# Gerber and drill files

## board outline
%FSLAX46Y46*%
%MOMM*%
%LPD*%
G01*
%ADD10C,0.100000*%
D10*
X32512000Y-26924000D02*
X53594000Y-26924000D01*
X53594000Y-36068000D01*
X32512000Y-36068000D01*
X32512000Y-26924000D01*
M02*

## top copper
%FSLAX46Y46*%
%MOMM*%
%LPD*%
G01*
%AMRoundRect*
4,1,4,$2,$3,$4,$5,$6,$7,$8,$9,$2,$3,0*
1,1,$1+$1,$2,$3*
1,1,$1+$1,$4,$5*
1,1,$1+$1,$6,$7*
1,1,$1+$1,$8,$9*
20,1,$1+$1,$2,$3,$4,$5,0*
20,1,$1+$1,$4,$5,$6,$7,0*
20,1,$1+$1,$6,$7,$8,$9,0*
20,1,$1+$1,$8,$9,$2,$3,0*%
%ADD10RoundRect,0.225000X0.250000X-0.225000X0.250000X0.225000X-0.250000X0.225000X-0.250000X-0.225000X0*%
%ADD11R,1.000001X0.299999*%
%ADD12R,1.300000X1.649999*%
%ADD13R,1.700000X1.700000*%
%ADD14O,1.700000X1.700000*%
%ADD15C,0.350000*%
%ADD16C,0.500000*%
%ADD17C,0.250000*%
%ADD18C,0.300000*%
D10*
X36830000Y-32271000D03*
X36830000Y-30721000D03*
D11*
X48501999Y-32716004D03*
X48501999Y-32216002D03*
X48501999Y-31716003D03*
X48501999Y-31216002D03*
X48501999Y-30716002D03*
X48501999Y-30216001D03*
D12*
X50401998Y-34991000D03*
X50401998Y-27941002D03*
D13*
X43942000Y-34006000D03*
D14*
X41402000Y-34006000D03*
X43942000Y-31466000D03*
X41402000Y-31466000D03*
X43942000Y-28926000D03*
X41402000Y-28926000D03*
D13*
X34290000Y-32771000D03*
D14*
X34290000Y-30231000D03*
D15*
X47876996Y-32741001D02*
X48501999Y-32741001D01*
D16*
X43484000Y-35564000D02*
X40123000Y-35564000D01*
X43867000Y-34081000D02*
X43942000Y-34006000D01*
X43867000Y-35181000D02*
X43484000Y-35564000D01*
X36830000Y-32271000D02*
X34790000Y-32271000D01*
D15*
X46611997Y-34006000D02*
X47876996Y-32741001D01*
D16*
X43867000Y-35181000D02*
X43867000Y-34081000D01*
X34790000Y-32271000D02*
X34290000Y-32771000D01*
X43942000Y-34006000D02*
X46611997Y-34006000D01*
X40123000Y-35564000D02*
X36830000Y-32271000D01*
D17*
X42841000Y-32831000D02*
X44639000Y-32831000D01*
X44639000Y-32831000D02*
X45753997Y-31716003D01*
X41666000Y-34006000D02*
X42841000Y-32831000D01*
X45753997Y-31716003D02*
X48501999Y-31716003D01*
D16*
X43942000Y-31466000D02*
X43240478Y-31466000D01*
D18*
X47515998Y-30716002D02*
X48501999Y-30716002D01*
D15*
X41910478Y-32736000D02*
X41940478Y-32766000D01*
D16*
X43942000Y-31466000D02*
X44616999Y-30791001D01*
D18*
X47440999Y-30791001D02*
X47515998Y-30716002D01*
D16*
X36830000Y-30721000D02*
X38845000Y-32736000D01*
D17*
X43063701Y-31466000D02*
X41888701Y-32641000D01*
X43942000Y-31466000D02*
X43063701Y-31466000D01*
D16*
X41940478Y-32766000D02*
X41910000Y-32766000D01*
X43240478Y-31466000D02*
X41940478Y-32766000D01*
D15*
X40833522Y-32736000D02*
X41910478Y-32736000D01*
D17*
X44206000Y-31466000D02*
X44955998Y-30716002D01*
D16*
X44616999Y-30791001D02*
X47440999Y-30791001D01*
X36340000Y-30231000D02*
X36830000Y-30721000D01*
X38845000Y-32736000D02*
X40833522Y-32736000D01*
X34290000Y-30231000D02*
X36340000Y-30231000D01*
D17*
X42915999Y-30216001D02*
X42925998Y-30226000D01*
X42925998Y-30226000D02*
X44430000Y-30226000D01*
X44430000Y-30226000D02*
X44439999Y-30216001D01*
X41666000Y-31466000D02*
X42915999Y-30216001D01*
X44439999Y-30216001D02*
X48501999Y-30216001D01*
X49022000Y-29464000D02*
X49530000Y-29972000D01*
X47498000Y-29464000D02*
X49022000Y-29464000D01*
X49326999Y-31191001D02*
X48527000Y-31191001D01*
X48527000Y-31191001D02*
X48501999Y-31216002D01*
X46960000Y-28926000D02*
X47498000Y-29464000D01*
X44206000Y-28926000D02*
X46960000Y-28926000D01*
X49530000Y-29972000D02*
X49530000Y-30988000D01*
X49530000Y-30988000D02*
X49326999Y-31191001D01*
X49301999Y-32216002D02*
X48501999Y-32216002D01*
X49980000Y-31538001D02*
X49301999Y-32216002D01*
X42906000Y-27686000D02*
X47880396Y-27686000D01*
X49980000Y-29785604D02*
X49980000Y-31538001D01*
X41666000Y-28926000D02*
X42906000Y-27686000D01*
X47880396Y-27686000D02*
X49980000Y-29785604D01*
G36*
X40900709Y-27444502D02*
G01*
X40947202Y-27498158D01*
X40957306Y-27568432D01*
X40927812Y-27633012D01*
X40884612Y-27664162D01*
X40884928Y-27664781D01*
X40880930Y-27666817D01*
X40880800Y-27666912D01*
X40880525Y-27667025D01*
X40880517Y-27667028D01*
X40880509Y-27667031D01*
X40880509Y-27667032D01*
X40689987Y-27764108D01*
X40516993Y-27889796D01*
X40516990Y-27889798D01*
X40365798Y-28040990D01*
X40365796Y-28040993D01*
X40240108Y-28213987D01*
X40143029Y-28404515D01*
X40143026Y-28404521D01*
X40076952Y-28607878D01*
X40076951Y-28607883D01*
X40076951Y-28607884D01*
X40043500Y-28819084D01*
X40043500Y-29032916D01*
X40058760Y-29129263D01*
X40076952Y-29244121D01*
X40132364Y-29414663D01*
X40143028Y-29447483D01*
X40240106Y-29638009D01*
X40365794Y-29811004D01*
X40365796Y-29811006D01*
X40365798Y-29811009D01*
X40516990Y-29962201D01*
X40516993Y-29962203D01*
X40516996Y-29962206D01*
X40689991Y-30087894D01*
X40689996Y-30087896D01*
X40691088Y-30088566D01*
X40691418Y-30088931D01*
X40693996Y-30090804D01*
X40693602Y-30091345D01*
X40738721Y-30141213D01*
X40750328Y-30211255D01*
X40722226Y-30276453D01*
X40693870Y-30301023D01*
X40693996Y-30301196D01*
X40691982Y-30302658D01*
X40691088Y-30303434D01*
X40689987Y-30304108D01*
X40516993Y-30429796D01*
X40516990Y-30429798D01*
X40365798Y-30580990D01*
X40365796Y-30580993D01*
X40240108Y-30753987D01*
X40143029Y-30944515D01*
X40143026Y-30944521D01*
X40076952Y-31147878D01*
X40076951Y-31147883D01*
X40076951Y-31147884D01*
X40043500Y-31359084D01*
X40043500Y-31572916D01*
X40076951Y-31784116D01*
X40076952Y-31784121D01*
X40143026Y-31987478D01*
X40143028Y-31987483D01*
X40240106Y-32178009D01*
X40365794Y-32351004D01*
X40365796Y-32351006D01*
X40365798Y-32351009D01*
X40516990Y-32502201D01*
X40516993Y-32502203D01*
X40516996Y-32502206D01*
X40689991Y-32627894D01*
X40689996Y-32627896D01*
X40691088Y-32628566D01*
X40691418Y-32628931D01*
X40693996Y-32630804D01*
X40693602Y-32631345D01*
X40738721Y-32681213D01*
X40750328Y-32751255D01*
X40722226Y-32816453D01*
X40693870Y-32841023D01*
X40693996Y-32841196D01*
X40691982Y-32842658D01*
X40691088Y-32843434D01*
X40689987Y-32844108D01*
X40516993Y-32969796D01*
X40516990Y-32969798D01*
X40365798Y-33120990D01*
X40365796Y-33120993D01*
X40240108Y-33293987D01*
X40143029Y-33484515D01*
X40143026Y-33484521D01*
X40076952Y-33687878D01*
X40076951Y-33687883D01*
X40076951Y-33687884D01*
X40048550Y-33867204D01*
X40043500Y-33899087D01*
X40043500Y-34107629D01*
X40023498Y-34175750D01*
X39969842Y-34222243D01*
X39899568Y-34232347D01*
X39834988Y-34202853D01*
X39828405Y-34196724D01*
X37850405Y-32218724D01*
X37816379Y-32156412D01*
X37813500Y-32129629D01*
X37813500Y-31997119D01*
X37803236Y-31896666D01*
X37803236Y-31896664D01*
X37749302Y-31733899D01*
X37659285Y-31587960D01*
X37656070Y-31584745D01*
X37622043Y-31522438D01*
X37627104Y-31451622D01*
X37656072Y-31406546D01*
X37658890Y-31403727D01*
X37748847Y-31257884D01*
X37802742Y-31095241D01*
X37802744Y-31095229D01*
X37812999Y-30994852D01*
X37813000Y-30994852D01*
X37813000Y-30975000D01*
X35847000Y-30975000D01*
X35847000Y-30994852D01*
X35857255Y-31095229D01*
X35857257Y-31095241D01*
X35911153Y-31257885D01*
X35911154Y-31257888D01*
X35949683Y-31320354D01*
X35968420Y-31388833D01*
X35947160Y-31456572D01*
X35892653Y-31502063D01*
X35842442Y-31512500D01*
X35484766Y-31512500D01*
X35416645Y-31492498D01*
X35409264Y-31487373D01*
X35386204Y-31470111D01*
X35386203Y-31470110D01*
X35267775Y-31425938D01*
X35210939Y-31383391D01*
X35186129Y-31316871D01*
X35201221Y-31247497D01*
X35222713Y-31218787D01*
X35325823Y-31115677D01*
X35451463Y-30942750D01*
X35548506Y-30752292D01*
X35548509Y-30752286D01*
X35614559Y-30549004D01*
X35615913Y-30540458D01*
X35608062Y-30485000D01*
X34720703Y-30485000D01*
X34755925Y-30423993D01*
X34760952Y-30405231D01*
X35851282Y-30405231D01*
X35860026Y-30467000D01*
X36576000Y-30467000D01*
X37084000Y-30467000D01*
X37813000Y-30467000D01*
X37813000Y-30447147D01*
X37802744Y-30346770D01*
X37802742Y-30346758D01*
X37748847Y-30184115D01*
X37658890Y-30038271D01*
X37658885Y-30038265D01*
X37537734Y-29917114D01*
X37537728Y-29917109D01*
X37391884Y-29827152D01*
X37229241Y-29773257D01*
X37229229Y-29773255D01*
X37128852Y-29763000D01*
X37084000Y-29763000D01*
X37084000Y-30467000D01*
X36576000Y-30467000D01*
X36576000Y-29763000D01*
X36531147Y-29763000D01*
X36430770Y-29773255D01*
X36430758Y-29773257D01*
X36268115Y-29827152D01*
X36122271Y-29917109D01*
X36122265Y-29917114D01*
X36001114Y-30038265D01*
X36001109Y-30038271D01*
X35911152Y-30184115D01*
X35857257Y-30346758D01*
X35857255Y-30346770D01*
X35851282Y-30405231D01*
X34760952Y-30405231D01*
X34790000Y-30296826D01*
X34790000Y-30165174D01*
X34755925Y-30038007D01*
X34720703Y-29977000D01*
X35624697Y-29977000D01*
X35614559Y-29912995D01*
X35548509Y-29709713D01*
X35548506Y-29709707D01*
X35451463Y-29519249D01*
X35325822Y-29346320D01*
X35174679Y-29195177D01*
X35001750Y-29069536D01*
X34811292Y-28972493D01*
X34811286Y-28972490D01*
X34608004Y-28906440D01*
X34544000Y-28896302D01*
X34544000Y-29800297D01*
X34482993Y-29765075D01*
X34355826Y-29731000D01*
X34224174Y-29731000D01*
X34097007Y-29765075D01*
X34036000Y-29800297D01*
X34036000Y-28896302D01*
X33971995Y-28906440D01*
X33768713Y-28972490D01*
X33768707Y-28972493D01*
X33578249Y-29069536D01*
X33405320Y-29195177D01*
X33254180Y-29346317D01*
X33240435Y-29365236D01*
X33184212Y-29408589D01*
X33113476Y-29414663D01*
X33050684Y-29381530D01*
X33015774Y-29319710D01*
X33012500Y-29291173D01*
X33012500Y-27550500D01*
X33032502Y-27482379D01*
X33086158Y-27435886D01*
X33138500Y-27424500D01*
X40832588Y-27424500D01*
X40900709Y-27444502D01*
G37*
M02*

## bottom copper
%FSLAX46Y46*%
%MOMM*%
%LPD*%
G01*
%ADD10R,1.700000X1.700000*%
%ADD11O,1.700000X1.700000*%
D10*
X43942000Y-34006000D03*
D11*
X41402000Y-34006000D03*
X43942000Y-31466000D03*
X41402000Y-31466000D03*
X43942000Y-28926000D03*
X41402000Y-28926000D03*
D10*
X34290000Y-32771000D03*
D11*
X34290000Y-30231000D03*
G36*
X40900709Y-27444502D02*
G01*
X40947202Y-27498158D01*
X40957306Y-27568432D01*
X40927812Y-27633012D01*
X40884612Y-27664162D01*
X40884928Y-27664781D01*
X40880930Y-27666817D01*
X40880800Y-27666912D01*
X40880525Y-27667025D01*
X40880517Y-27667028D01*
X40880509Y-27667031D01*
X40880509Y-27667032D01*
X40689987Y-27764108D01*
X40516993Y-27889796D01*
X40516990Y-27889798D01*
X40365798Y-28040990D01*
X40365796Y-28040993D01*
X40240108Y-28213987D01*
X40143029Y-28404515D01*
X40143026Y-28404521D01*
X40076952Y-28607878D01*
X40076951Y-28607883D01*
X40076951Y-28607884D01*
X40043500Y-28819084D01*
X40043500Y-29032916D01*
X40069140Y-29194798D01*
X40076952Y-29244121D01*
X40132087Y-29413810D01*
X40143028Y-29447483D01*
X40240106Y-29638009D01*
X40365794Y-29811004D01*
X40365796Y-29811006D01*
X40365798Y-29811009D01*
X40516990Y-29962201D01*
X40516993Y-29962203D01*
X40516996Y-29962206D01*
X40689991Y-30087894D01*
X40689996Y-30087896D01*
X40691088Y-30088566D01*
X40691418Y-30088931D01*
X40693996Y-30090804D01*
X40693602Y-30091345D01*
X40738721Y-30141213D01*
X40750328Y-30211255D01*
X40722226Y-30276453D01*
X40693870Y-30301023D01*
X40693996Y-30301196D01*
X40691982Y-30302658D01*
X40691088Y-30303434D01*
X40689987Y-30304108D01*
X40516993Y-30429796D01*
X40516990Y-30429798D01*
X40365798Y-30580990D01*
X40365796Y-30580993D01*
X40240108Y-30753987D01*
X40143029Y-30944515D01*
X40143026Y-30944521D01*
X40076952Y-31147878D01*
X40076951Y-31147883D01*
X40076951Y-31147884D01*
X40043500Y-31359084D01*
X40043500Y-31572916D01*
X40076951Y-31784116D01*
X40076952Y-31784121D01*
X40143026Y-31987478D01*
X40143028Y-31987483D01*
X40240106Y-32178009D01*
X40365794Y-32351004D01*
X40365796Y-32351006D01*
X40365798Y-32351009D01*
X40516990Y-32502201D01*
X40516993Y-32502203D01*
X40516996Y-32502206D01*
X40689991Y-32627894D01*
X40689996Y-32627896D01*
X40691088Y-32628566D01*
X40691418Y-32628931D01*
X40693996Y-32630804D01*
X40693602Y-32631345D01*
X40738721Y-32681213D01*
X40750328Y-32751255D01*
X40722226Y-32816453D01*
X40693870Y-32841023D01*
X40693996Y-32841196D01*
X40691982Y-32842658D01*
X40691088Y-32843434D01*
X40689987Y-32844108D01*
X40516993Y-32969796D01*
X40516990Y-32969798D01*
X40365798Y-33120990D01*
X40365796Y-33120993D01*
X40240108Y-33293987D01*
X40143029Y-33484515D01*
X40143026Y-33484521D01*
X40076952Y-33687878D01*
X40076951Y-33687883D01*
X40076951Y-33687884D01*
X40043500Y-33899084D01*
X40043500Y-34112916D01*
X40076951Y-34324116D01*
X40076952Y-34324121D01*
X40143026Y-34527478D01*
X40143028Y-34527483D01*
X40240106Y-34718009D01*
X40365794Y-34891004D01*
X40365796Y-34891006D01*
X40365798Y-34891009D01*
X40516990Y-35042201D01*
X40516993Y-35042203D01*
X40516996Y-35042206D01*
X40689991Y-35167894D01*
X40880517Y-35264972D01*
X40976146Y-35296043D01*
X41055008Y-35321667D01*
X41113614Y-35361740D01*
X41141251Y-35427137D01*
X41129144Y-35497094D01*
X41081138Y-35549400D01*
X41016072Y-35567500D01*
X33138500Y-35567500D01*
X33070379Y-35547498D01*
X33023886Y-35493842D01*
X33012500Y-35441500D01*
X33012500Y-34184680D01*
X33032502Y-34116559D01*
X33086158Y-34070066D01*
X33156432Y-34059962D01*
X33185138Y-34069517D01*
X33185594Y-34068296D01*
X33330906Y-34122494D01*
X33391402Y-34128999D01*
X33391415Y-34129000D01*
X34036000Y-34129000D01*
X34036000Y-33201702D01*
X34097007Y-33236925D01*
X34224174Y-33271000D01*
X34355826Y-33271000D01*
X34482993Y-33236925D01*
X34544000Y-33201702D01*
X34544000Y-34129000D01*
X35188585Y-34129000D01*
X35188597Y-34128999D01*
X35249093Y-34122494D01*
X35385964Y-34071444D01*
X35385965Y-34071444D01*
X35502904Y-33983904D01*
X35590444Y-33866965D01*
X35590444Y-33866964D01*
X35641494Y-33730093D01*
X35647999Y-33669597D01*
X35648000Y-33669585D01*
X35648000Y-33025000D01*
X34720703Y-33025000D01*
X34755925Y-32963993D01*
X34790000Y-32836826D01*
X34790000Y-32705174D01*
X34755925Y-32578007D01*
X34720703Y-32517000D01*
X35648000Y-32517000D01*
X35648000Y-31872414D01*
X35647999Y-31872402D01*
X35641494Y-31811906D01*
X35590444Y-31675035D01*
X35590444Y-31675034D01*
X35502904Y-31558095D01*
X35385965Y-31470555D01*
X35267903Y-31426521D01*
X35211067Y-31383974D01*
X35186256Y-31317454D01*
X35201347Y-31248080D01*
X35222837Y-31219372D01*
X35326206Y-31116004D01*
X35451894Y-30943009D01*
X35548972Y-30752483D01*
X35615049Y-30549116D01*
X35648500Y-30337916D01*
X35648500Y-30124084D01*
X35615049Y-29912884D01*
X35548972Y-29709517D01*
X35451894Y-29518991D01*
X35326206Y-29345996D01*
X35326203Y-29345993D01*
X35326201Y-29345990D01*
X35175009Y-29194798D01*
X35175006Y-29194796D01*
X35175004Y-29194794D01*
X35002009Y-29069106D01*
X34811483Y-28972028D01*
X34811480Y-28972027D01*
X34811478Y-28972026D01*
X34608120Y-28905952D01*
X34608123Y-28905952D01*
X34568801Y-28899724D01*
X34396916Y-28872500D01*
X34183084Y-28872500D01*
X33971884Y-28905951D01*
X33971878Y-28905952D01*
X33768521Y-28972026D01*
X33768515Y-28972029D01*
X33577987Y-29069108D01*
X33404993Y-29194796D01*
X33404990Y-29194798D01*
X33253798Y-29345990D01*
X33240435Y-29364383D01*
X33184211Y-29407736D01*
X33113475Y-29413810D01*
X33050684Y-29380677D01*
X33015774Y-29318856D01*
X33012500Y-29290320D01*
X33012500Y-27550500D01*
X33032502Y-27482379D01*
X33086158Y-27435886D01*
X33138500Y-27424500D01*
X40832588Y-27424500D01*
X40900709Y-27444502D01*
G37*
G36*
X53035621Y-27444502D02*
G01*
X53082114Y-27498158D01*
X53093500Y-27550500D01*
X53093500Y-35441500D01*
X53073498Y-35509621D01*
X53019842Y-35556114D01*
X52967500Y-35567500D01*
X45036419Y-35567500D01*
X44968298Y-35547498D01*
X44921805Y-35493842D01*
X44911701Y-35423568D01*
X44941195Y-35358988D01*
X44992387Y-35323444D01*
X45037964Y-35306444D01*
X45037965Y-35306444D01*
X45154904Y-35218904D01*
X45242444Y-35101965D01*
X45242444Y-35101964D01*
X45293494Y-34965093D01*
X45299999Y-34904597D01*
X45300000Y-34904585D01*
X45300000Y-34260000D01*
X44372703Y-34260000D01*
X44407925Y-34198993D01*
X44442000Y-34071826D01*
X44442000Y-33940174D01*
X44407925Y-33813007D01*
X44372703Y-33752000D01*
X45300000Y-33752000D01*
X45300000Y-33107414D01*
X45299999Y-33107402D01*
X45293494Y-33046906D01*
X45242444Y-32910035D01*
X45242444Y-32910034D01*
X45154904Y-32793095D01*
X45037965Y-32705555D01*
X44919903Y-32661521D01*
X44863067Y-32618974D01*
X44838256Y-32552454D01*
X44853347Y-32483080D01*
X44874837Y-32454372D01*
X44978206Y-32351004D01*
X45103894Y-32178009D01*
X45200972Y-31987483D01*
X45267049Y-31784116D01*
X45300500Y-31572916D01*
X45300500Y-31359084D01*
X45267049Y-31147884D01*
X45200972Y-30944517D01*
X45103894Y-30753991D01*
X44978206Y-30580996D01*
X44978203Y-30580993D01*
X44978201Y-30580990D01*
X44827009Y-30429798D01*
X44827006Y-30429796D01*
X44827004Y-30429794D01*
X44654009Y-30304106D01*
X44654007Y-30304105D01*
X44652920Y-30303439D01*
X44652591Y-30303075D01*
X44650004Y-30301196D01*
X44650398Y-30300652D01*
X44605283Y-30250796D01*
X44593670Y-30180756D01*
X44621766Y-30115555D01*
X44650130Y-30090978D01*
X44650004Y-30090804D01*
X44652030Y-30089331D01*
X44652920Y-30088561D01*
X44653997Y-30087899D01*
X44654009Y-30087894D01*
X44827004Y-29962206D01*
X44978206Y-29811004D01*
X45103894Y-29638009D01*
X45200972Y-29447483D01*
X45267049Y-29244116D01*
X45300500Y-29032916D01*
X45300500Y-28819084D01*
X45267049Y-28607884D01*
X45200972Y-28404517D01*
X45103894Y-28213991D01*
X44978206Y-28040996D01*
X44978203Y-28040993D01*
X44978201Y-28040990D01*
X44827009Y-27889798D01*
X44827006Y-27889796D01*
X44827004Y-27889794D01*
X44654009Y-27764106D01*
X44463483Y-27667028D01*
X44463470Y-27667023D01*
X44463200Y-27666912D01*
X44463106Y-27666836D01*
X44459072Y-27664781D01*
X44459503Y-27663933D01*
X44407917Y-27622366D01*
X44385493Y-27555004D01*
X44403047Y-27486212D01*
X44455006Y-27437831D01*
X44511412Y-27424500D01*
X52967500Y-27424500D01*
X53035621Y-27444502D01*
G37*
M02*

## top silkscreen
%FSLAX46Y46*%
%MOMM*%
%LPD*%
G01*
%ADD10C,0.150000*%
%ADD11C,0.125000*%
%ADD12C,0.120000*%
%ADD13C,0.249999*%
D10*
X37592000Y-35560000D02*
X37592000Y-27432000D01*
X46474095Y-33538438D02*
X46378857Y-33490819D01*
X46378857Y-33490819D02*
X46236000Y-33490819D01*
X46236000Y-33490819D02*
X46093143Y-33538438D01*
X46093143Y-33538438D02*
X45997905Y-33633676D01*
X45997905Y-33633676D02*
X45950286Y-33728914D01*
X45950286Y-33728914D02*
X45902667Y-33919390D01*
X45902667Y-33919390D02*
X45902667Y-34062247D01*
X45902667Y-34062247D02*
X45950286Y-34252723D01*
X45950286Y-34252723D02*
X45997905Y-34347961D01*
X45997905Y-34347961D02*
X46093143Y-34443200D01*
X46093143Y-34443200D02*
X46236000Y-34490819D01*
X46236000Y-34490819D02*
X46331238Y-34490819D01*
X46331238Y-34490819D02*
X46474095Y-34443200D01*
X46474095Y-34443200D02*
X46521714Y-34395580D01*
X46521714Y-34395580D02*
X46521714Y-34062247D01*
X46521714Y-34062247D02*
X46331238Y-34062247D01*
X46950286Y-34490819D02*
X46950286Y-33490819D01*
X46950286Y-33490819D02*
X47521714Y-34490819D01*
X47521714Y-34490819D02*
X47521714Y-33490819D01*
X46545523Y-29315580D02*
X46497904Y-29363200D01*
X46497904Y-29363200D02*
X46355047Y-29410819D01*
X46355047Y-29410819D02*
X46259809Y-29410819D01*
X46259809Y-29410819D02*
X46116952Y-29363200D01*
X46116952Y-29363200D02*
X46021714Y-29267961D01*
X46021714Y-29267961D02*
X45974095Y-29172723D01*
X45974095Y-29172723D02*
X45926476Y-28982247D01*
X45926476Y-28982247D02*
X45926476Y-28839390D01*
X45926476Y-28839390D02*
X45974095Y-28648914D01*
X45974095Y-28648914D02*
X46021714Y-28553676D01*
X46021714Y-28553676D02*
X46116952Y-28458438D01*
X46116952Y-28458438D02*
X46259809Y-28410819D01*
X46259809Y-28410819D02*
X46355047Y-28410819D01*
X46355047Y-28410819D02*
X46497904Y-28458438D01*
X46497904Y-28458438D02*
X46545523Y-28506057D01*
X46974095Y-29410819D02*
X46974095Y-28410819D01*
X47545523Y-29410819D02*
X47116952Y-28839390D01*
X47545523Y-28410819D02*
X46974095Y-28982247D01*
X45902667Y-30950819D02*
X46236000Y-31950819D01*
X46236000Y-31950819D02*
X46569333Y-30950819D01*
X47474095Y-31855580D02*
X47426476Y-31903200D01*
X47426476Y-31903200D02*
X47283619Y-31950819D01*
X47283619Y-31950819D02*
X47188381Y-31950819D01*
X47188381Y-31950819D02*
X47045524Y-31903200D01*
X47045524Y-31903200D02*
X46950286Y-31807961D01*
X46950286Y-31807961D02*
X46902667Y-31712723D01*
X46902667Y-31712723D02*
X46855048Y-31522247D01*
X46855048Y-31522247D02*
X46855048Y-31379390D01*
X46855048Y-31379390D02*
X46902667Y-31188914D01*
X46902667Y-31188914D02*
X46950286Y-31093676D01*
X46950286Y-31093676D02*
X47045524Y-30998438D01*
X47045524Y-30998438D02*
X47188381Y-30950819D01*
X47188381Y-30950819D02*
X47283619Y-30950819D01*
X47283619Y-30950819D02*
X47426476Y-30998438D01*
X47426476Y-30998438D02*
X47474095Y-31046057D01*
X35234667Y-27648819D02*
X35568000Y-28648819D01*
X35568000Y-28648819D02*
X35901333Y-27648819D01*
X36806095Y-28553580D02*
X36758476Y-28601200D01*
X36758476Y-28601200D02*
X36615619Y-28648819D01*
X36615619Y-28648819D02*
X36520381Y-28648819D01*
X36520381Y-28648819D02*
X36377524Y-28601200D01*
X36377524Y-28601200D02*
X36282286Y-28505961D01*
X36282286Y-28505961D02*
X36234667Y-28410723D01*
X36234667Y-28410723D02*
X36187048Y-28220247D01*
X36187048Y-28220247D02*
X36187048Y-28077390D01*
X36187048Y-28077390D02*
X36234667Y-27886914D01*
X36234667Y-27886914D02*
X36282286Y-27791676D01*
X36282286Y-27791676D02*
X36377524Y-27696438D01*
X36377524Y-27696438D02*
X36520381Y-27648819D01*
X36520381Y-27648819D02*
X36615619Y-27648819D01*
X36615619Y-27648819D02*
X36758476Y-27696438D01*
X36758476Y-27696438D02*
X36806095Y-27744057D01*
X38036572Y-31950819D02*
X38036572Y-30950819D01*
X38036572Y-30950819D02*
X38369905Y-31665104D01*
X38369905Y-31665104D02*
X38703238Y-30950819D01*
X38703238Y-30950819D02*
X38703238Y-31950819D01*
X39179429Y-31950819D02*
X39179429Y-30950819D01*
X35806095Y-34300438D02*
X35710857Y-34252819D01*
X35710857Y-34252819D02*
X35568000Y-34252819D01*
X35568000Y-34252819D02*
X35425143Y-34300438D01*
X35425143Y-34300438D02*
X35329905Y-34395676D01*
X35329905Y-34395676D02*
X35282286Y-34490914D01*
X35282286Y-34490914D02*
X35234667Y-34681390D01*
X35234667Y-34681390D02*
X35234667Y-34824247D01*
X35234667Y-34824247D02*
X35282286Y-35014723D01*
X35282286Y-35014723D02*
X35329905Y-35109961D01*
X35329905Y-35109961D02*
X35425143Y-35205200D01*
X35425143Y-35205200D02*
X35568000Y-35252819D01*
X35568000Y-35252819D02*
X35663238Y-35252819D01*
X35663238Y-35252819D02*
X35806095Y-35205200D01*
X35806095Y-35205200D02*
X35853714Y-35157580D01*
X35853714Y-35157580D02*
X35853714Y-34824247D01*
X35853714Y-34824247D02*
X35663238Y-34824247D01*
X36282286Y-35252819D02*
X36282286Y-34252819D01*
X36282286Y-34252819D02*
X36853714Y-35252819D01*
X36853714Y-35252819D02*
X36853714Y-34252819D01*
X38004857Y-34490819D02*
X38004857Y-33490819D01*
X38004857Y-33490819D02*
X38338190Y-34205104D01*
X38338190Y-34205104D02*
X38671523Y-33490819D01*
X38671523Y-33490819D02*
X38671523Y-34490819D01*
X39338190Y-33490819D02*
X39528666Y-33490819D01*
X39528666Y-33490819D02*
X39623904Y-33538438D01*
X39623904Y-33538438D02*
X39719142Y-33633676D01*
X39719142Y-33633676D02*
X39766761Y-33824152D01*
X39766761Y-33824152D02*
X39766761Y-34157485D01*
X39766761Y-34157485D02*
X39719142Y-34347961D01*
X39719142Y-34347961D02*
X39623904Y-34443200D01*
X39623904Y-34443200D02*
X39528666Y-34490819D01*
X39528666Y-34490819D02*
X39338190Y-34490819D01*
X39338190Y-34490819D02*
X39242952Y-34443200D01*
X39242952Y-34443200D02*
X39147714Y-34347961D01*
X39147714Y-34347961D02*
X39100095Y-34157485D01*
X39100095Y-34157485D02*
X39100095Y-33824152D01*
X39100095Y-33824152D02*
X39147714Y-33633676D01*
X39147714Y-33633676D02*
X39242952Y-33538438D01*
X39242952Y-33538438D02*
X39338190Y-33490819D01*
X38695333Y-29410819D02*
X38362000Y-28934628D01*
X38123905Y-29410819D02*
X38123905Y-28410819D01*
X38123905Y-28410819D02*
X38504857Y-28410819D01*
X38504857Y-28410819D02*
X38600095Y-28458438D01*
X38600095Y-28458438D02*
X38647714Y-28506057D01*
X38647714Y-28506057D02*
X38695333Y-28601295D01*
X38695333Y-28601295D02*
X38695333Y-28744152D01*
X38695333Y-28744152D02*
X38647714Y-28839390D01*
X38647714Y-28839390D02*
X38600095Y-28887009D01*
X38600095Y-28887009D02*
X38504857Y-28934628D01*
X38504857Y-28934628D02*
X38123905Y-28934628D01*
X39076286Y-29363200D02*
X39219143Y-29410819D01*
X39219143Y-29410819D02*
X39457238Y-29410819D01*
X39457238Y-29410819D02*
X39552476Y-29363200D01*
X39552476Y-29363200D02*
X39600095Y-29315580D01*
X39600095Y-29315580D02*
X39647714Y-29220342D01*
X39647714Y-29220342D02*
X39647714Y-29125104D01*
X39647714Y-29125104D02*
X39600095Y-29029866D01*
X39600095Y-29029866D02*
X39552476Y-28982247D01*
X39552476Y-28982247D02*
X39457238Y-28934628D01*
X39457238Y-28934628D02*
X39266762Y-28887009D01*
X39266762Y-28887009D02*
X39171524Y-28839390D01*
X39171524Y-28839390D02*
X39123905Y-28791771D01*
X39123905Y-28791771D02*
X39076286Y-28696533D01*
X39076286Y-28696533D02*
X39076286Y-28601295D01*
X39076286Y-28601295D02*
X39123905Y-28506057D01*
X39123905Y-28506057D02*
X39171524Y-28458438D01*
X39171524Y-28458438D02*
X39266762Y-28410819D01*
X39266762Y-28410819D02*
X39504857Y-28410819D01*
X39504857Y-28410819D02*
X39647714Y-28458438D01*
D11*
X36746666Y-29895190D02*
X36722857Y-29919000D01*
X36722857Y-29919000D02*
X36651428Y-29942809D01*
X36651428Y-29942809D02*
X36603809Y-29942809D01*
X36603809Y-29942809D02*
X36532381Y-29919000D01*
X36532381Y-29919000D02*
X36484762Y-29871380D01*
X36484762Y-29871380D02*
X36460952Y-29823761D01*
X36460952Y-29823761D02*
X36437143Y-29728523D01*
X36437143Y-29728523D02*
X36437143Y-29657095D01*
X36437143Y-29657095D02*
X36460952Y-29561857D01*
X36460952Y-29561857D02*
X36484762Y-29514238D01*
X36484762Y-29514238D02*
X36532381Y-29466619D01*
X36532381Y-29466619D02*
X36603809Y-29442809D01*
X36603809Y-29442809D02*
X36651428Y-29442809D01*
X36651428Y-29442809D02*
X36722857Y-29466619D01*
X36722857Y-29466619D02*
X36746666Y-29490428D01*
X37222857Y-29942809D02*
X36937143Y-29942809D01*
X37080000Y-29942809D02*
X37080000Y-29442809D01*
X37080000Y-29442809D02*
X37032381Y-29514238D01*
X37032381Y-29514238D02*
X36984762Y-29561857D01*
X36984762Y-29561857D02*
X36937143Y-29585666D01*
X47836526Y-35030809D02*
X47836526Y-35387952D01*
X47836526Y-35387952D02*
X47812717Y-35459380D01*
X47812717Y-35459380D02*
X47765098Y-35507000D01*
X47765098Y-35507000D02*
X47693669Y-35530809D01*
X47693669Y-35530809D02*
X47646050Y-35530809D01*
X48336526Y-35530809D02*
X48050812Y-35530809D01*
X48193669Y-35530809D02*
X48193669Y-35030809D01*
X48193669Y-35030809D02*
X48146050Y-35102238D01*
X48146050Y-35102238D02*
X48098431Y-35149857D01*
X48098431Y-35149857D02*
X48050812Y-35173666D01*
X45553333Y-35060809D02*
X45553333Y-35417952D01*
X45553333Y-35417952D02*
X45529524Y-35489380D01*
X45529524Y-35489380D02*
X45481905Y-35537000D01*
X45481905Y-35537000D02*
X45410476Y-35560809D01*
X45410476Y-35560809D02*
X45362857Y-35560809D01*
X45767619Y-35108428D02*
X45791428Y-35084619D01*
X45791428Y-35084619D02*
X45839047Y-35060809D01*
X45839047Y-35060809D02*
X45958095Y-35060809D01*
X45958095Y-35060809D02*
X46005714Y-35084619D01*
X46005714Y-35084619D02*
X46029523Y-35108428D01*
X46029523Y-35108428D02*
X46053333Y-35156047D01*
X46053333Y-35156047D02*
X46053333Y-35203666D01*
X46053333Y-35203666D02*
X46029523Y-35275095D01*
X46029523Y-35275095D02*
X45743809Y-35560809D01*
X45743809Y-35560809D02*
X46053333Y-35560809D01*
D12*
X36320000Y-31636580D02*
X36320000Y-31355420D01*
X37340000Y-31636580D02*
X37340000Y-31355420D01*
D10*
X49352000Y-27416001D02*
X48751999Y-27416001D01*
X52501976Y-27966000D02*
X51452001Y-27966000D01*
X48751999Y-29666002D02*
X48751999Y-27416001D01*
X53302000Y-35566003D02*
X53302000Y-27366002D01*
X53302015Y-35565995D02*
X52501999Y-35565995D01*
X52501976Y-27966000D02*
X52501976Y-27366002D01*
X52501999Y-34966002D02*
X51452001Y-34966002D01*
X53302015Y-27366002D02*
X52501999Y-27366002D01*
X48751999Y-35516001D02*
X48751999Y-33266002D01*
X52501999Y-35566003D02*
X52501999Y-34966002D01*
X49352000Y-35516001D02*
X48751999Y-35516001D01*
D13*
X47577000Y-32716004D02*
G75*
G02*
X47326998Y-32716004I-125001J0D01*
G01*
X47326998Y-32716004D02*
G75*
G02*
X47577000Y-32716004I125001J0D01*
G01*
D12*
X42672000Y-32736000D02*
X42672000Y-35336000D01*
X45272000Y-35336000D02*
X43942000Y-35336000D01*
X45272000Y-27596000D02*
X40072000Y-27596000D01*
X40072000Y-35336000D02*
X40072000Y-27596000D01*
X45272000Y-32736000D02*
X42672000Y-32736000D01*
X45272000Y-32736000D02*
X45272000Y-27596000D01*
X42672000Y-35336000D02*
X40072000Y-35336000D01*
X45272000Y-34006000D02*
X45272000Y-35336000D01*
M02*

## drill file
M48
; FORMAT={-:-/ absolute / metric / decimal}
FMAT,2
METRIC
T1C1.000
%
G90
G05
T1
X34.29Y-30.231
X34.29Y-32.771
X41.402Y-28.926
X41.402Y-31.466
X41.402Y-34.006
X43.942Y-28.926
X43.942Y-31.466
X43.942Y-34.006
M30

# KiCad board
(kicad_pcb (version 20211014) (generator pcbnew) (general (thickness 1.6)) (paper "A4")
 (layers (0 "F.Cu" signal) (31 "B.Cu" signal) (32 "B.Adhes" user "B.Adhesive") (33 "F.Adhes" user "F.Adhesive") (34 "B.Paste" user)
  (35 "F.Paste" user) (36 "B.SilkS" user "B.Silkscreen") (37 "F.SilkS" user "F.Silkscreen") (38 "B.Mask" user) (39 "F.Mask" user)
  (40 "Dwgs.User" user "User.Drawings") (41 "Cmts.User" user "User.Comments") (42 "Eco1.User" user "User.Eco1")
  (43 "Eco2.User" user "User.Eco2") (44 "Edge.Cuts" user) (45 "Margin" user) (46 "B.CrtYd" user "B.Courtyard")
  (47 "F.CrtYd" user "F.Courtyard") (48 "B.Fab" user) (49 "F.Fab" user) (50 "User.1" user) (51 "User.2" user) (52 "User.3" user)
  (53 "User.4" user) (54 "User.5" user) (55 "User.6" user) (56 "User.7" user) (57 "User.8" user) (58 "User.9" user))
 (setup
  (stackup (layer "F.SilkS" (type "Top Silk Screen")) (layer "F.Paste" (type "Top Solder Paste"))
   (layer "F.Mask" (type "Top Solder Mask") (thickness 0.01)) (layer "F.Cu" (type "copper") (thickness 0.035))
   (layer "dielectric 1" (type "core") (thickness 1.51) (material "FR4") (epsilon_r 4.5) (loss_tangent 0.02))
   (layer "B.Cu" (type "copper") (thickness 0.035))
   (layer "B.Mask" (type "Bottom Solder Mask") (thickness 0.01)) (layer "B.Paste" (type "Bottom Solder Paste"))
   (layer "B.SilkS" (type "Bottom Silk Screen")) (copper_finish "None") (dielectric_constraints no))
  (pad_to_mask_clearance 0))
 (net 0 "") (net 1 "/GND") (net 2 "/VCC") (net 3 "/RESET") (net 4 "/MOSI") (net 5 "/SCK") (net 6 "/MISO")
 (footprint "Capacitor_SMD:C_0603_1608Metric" (layer "F.Cu") (at 36.83 31.496 90)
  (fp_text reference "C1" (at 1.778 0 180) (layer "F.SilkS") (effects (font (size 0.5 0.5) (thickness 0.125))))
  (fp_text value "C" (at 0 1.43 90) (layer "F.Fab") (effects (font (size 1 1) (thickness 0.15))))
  (fp_line (start -0.14058 -0.51) (end 0.14058 -0.51) (layer "F.SilkS") (width 0.12))
  (fp_line (start -0.14058 0.51) (end 0.14058 0.51) (layer "F.SilkS") (width 0.12))
  (pad "1" smd roundrect (at -0.775 0 90) (size 0.9 0.95) (layers "F.Cu" "F.Paste" "F.Mask") (roundrect_rratio 0.25) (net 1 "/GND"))
  (pad "2" smd roundrect (at 0.775 0 90) (size 0.9 0.95) (layers "F.Cu" "F.Paste" "F.Mask") (roundrect_rratio 0.25) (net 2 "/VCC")))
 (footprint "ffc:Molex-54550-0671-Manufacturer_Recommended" (layer "F.Cu") (at 49.452 31.466001 90)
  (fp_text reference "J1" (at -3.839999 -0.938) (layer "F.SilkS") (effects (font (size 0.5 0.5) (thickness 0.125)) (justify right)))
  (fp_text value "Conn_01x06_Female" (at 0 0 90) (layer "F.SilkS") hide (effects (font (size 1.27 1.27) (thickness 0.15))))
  (fp_line (start 4.05 -0.1) (end 4.05 -0.700001) (layer "F.SilkS") (width 0.15))
  (fp_line (start 3.500001 3.049976) (end 3.500001 2.000001) (layer "F.SilkS") (width 0.15))
  (fp_line (start 1.799999 -0.700001) (end 4.05 -0.700001) (layer "F.SilkS") (width 0.15))
  (fp_line (start -4.100002 3.85) (end 4.099999 3.85) (layer "F.SilkS") (width 0.15))
  (fp_line (start -4.099994 3.850015) (end -4.099994 3.049999) (layer "F.SilkS") (width 0.15))
  (fp_line (start 3.500001 3.049976) (end 4.099999 3.049976) (layer "F.SilkS") (width 0.15))
  (fp_line (start -3.500001 3.049999) (end -3.500001 2.000001) (layer "F.SilkS") (width 0.15))
  (fp_line (start 4.099999 3.850015) (end 4.099999 3.049999) (layer "F.SilkS") (width 0.15))
  (fp_line (start -4.05 -0.700001) (end -1.800001 -0.700001) (layer "F.SilkS") (width 0.15))
  (fp_line (start -4.100002 3.049999) (end -3.500001 3.049999) (layer "F.SilkS") (width 0.15))
  (fp_line (start -4.05 -0.1) (end -4.05 -0.700001) (layer "F.SilkS") (width 0.15))
  (fp_circle (center -1.250003 -2.000001) (end -1.125002 -2.000001) (layer "F.SilkS") (width 0.249999) (fill none))
  (pad "1" smd rect locked (at -1.250003 -0.950001 90) (size 0.299999 1.000001) (layers "F.Cu" "F.Paste" "F.Mask") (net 1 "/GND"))
  (pad "2" smd rect locked (at -0.750001 -0.950001 90) (size 0.299999 1.000001) (layers "F.Cu" "F.Paste" "F.Mask") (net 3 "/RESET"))
  (pad "3" smd rect locked (at -0.250002 -0.950001 90) (size 0.299999 1.000001) (layers "F.Cu" "F.Paste" "F.Mask") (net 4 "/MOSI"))
  (pad "4" smd rect locked (at 0.249999 -0.950001 90) (size 0.299999 1.000001) (layers "F.Cu" "F.Paste" "F.Mask") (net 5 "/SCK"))
  (pad "5" smd rect locked (at 0.749999 -0.950001 90) (size 0.299999 1.000001) (layers "F.Cu" "F.Paste" "F.Mask") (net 2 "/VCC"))
  (pad "6" smd rect locked (at 1.25 -0.950001 90) (size 0.299999 1.000001) (layers "F.Cu" "F.Paste" "F.Mask") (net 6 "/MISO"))
  (pad "MP1" smd rect locked (at -3.524999 0.949998 90) (size 1.649999 1.3) (layers "F.Cu" "F.Paste" "F.Mask"))
  (pad "MP2" smd rect locked (at 3.524999 0.949998 90) (size 1.649999 1.3) (layers "F.Cu" "F.Paste" "F.Mask")))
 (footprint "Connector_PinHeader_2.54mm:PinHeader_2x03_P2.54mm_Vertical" (layer "F.Cu") (at 43.942 34.006 180)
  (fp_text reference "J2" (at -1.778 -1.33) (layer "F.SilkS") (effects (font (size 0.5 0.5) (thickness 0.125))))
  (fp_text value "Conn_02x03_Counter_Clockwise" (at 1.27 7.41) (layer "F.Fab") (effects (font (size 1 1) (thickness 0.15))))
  (fp_line (start 1.27 1.27) (end 1.27 -1.33) (layer "F.SilkS") (width 0.12))
  (fp_line (start -1.33 -1.33) (end 0 -1.33) (layer "F.SilkS") (width 0.12))
  (fp_line (start -1.33 6.41) (end 3.87 6.41) (layer "F.SilkS") (width 0.12))
  (fp_line (start 3.87 -1.33) (end 3.87 6.41) (layer "F.SilkS") (width 0.12))
  (fp_line (start -1.33 1.27) (end 1.27 1.27) (layer "F.SilkS") (width 0.12))
  (fp_line (start -1.33 1.27) (end -1.33 6.41) (layer "F.SilkS") (width 0.12))
  (fp_line (start 1.27 -1.33) (end 3.87 -1.33) (layer "F.SilkS") (width 0.12))
  (fp_line (start -1.33 0) (end -1.33 -1.33) (layer "F.SilkS") (width 0.12))
  (pad "1" thru_hole rect (at 0 0 180) (size 1.7 1.7) (drill 1) (layers *.Cu *.Mask) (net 1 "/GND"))
  (pad "2" thru_hole oval (at 2.54 0 180) (size 1.7 1.7) (drill 1) (layers *.Cu *.Mask) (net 4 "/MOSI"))
  (pad "3" thru_hole oval (at 0 2.54 180) (size 1.7 1.7) (drill 1) (layers *.Cu *.Mask) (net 2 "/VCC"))
  (pad "4" thru_hole oval (at 2.54 2.54 180) (size 1.7 1.7) (drill 1) (layers *.Cu *.Mask) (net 6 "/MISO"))
  (pad "5" thru_hole oval (at 0 5.08 180) (size 1.7 1.7) (drill 1) (layers *.Cu *.Mask) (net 5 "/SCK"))
  (pad "6" thru_hole oval (at 2.54 5.08 180) (size 1.7 1.7) (drill 1) (layers *.Cu *.Mask) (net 3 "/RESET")))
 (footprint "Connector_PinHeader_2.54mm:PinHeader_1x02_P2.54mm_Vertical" (layer "B.Cu") (at 34.29 32.771)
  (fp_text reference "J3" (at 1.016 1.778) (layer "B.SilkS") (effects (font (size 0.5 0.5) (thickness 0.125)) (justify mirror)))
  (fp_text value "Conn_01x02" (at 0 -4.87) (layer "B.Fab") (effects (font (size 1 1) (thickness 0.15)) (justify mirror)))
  (pad "1" thru_hole rect (at 0 0) (size 1.7 1.7) (drill 1) (layers *.Cu *.Mask) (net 1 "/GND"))
  (pad "2" thru_hole oval (at 0 -2.54) (size 1.7 1.7) (drill 1) (layers *.Cu *.Mask) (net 2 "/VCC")))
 (gr_line (start 37.592 35.56) (end 37.592 27.432) (layer "F.SilkS") (width 0.15))
 (gr_rect (start 32.512 26.924) (end 53.594 36.068) (layer "Edge.Cuts") (width 0.1) (fill none))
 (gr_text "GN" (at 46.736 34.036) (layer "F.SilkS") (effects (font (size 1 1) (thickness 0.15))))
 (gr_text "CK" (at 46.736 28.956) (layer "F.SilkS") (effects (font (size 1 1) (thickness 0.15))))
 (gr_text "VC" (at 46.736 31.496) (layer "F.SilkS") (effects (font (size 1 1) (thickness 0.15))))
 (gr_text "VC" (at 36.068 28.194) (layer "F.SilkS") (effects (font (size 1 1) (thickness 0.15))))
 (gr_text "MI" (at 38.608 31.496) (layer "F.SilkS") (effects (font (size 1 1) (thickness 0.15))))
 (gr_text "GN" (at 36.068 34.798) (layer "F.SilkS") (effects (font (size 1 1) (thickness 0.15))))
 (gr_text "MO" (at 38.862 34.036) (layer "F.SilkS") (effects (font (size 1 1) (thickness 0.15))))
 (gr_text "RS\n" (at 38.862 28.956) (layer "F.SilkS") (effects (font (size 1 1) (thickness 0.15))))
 (segment (start 47.876996 32.741001) (end 48.501999 32.741001) (width 0.35) (layer "F.Cu") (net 1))
 (segment (start 43.484 35.564) (end 40.123 35.564) (width 0.5) (layer "F.Cu") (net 1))
 (segment (start 43.867 34.081) (end 43.942 34.006) (width 0.5) (layer "F.Cu") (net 1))
 (segment (start 43.867 35.181) (end 43.484 35.564) (width 0.5) (layer "F.Cu") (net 1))
 (segment (start 36.83 32.271) (end 34.79 32.271) (width 0.5) (layer "F.Cu") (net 1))
 (segment (start 46.611997 34.006) (end 47.876996 32.741001) (width 0.35) (layer "F.Cu") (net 1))
 (segment (start 43.867 35.181) (end 43.867 34.081) (width 0.5) (layer "F.Cu") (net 1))
 (segment (start 34.79 32.271) (end 34.29 32.771) (width 0.5) (layer "F.Cu") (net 1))
 (segment (start 43.942 34.006) (end 46.611997 34.006) (width 0.5) (layer "F.Cu") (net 1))
 (segment (start 40.123 35.564) (end 36.83 32.271) (width 0.5) (layer "F.Cu") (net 1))
 (segment (start 42.841 32.831) (end 44.639 32.831) (width 0.25) (layer "F.Cu") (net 4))
 (segment (start 44.639 32.831) (end 45.753997 31.716003) (width 0.25) (layer "F.Cu") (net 4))
 (segment (start 41.666 34.006) (end 42.841 32.831) (width 0.25) (layer "F.Cu") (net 4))
 (segment (start 45.753997 31.716003) (end 48.501999 31.716003) (width 0.25) (layer "F.Cu") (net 4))
 (segment (start 43.942 31.466) (end 43.240478 31.466) (width 0.5) (layer "F.Cu") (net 2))
 (segment (start 47.515998 30.716002) (end 48.501999 30.716002) (width 0.3) (layer "F.Cu") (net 2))
 (segment (start 41.910478 32.736) (end 41.940478 32.766) (width 0.35) (layer "F.Cu") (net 2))
 (segment (start 43.942 31.466) (end 44.616999 30.791001) (width 0.5) (layer "F.Cu") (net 2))
 (segment (start 47.440999 30.791001) (end 47.515998 30.716002) (width 0.3) (layer "F.Cu") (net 2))
 (segment (start 36.83 30.721) (end 38.845 32.736) (width 0.5) (layer "F.Cu") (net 2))
 (segment (start 43.063701 31.466) (end 41.888701 32.641) (width 0.25) (layer "F.Cu") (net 2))
 (segment (start 43.942 31.466) (end 43.063701 31.466) (width 0.25) (layer "F.Cu") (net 2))
 (segment (start 41.940478 32.766) (end 41.91 32.766) (width 0.5) (layer "F.Cu") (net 2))
 (segment (start 43.240478 31.466) (end 41.940478 32.766) (width 0.5) (layer "F.Cu") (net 2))
 (segment (start 40.833522 32.736) (end 41.910478 32.736) (width 0.35) (layer "F.Cu") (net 2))
 (segment (start 44.206 31.466) (end 44.955998 30.716002) (width 0.25) (layer "F.Cu") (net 2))
 (segment (start 44.616999 30.791001) (end 47.440999 30.791001) (width 0.5) (layer "F.Cu") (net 2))
 (segment (start 36.34 30.231) (end 36.83 30.721) (width 0.5) (layer "F.Cu") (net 2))
 (segment (start 38.845 32.736) (end 40.833522 32.736) (width 0.5) (layer "F.Cu") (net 2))
 (segment (start 34.29 30.231) (end 36.34 30.231) (width 0.5) (layer "F.Cu") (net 2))
 (segment (start 42.915999 30.216001) (end 42.925998 30.226) (width 0.25) (layer "F.Cu") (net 6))
 (segment (start 42.925998 30.226) (end 44.43 30.226) (width 0.25) (layer "F.Cu") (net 6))
 (segment (start 44.43 30.226) (end 44.439999 30.216001) (width 0.25) (layer "F.Cu") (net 6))
 (segment (start 41.666 31.466) (end 42.915999 30.216001) (width 0.25) (layer "F.Cu") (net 6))
 (segment (start 44.439999 30.216001) (end 48.501999 30.216001) (width 0.25) (layer "F.Cu") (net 6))
 (segment (start 49.022 29.464) (end 49.53 29.972) (width 0.25) (layer "F.Cu") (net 5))
 (segment (start 47.498 29.464) (end 49.022 29.464) (width 0.25) (layer "F.Cu") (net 5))
 (segment (start 49.326999 31.191001) (end 48.527 31.191001) (width 0.25) (layer "F.Cu") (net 5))
 (segment (start 48.527 31.191001) (end 48.501999 31.216002) (width 0.25) (layer "F.Cu") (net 5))
 (segment (start 46.96 28.926) (end 47.498 29.464) (width 0.25) (layer "F.Cu") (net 5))
 (segment (start 44.206 28.926) (end 46.96 28.926) (width 0.25) (layer "F.Cu") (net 5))
 (segment (start 49.53 29.972) (end 49.53 30.988) (width 0.25) (layer "F.Cu") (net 5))
 (segment (start 49.53 30.988) (end 49.326999 31.191001) (width 0.25) (layer "F.Cu") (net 5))
 (segment (start 49.301999 32.216002) (end 48.501999 32.216002) (width 0.25) (layer "F.Cu") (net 3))
 (segment (start 49.98 31.538001) (end 49.301999 32.216002) (width 0.25) (layer "F.Cu") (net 3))
 (segment (start 42.906 27.686) (end 47.880396 27.686) (width 0.25) (layer "F.Cu") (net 3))
 (segment (start 49.98 29.785604) (end 49.98 31.538001) (width 0.25) (layer "F.Cu") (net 3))
 (segment (start 41.666 28.926) (end 42.906 27.686) (width 0.25) (layer "F.Cu") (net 3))
 (segment (start 47.880396 27.686) (end 49.98 29.785604) (width 0.25) (layer "F.Cu") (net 3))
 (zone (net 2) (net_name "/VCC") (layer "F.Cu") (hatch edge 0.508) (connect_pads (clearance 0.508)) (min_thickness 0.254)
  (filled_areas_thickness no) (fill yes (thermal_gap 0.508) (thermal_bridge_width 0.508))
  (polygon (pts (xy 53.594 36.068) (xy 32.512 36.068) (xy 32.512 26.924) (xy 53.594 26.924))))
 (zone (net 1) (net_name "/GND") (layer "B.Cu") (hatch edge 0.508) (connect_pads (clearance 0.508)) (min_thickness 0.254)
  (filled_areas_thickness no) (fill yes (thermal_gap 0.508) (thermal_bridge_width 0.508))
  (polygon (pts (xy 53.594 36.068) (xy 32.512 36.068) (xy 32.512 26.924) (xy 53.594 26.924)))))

